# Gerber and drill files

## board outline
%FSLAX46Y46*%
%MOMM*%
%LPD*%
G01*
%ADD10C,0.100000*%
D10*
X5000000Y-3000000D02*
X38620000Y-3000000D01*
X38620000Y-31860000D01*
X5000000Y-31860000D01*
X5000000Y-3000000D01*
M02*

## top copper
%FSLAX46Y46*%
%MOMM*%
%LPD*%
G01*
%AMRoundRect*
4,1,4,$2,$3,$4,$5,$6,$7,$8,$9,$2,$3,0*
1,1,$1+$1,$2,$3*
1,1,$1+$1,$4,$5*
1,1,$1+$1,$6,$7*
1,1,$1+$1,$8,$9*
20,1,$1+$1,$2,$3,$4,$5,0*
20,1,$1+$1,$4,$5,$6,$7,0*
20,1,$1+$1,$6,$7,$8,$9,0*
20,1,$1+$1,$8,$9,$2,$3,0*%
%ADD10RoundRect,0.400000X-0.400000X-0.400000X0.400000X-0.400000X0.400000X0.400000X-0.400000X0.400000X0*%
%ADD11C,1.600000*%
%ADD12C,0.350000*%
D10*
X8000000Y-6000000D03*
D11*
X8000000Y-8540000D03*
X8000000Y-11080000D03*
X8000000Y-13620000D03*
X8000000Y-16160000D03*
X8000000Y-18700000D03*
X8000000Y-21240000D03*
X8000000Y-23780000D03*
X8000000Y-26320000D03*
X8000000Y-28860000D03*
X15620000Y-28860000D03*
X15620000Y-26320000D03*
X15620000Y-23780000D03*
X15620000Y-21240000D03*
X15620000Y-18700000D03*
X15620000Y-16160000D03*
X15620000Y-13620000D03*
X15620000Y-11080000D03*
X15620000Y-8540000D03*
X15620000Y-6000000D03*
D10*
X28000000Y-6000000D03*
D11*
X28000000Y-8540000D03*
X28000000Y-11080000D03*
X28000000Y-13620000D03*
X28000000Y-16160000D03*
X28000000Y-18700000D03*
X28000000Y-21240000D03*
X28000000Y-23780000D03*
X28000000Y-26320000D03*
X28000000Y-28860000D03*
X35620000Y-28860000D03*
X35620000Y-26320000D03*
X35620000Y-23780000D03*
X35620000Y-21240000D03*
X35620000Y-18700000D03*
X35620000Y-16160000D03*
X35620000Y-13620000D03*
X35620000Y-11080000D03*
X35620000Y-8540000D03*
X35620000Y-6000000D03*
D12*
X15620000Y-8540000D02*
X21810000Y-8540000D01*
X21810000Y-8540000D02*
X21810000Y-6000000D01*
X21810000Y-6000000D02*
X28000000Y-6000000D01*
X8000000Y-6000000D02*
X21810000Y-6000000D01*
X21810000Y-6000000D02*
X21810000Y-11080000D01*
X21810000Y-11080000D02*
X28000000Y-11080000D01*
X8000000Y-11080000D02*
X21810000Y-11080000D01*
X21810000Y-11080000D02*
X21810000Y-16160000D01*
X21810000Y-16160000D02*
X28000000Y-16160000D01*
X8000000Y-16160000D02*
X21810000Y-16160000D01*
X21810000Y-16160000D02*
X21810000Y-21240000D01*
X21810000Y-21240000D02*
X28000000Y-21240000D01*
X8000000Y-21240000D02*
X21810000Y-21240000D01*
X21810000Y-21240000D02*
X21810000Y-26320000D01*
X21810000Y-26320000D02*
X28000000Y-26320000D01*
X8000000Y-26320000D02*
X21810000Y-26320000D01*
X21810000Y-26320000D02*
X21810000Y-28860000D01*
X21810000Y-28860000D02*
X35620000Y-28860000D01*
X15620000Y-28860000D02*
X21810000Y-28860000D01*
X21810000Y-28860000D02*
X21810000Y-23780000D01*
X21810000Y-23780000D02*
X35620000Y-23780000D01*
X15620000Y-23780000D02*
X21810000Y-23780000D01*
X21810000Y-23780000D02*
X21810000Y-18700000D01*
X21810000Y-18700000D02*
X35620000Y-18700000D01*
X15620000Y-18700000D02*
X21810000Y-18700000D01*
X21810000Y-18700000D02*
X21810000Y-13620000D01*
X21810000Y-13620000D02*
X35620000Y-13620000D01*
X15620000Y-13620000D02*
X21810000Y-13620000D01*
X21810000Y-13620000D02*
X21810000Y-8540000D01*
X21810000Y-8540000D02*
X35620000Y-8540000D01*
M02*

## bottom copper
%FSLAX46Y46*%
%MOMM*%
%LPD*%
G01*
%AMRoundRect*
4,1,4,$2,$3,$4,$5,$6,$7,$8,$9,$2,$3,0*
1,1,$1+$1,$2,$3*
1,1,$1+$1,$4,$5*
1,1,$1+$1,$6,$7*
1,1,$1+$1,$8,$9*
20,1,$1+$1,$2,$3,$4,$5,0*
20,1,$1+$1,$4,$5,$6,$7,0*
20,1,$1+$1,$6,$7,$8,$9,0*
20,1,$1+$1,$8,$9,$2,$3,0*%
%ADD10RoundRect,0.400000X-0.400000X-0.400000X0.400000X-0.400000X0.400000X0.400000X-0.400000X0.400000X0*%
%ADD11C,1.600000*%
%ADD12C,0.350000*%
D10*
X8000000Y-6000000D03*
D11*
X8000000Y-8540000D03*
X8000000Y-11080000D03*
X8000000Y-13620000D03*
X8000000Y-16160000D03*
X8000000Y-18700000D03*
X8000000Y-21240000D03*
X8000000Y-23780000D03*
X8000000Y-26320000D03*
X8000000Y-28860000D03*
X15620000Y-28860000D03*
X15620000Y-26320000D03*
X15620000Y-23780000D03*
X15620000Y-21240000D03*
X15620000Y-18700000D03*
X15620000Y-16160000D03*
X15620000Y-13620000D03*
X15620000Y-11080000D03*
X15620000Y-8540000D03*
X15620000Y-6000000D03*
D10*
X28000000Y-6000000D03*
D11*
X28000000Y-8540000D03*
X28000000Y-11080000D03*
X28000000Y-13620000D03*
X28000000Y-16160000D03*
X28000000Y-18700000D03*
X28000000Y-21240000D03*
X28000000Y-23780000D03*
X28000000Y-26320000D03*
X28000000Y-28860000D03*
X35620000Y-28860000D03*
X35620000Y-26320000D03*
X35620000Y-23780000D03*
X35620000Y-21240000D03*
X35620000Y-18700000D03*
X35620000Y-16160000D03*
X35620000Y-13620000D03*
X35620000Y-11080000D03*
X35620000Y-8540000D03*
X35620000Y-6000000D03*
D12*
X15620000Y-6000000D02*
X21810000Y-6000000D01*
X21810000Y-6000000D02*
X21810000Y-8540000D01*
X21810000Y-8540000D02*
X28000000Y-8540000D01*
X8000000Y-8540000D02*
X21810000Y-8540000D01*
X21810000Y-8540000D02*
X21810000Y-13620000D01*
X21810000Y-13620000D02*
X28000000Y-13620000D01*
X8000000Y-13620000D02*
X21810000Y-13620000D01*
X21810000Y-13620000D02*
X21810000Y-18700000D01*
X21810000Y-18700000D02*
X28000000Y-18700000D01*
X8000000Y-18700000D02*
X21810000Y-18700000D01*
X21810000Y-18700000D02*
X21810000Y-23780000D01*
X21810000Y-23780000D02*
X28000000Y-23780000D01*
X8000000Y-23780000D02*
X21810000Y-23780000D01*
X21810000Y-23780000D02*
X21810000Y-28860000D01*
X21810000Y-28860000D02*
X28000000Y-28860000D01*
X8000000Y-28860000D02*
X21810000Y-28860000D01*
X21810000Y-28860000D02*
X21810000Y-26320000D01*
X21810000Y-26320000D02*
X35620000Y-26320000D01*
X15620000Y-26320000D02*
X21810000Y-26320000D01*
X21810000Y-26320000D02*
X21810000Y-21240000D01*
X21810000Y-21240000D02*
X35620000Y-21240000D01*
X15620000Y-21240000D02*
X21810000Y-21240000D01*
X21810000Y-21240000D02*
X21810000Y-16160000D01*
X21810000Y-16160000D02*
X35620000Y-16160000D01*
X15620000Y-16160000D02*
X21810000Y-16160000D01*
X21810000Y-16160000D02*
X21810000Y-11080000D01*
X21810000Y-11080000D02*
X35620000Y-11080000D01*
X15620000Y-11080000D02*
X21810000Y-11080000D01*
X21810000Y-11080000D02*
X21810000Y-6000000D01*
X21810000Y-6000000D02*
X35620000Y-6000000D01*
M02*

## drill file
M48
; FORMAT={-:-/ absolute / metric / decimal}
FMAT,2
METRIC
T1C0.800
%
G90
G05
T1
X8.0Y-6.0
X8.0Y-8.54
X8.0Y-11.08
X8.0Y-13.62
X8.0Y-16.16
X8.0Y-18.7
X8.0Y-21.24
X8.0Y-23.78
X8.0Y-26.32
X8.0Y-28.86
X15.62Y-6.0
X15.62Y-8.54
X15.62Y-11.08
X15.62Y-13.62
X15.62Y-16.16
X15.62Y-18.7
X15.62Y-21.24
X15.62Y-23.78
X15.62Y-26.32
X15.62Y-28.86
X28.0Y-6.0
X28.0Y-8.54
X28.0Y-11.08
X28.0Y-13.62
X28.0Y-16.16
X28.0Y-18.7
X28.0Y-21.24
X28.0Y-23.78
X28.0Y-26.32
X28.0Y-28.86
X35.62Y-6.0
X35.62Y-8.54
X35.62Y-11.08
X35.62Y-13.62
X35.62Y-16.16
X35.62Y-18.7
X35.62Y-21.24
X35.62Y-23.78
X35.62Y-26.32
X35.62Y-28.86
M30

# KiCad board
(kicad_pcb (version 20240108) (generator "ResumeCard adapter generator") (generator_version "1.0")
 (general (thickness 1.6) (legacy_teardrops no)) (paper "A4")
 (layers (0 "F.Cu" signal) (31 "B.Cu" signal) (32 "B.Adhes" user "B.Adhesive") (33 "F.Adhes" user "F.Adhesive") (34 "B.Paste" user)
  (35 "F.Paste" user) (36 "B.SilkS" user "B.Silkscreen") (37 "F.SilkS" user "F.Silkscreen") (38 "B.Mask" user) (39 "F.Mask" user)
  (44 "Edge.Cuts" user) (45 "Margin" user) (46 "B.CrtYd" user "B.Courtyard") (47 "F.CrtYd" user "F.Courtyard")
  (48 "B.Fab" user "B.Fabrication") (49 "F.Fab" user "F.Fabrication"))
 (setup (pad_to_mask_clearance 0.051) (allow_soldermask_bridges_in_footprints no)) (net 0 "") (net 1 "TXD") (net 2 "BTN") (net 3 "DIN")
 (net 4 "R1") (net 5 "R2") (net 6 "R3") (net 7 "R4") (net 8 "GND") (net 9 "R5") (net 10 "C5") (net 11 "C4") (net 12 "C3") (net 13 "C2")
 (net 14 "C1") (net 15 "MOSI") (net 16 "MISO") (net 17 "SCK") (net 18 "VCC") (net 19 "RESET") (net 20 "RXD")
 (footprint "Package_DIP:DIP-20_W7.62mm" (layer "F.Cu") (at 8.0 6.0)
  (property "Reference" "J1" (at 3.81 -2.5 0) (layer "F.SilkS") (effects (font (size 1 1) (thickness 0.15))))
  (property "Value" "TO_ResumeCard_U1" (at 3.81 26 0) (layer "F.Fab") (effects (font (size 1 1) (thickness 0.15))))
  (pad "1" thru_hole roundrect (at 0.0 0.0) (size 1.6 1.6) (drill 0.8) (layers "*.Cu" "*.Mask") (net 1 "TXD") (roundrect_rratio 0.25))
  (pad "2" thru_hole circle (at 0.0 2.54) (size 1.6 1.6) (drill 0.8) (layers "*.Cu" "*.Mask") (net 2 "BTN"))
  (pad "3" thru_hole circle (at 0.0 5.08) (size 1.6 1.6) (drill 0.8) (layers "*.Cu" "*.Mask") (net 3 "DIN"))
  (pad "4" thru_hole circle (at 0.0 7.62) (size 1.6 1.6) (drill 0.8) (layers "*.Cu" "*.Mask") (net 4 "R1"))
  (pad "5" thru_hole circle (at 0.0 10.16) (size 1.6 1.6) (drill 0.8) (layers "*.Cu" "*.Mask") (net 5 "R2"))
  (pad "6" thru_hole circle (at 0.0 12.7) (size 1.6 1.6) (drill 0.8) (layers "*.Cu" "*.Mask") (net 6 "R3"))
  (pad "7" thru_hole circle (at 0.0 15.24) (size 1.6 1.6) (drill 0.8) (layers "*.Cu" "*.Mask") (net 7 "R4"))
  (pad "8" thru_hole circle (at 0.0 17.78) (size 1.6 1.6) (drill 0.8) (layers "*.Cu" "*.Mask") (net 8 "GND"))
  (pad "9" thru_hole circle (at 0.0 20.32) (size 1.6 1.6) (drill 0.8) (layers "*.Cu" "*.Mask") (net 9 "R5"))
  (pad "10" thru_hole circle (at 0.0 22.86) (size 1.6 1.6) (drill 0.8) (layers "*.Cu" "*.Mask") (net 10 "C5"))
  (pad "11" thru_hole circle (at 7.62 22.86) (size 1.6 1.6) (drill 0.8) (layers "*.Cu" "*.Mask") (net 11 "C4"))
  (pad "12" thru_hole circle (at 7.62 20.32) (size 1.6 1.6) (drill 0.8) (layers "*.Cu" "*.Mask") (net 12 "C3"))
  (pad "13" thru_hole circle (at 7.62 17.78) (size 1.6 1.6) (drill 0.8) (layers "*.Cu" "*.Mask") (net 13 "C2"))
  (pad "14" thru_hole circle (at 7.62 15.24) (size 1.6 1.6) (drill 0.8) (layers "*.Cu" "*.Mask") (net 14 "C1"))
  (pad "15" thru_hole circle (at 7.62 12.7) (size 1.6 1.6) (drill 0.8) (layers "*.Cu" "*.Mask") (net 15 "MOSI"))
  (pad "16" thru_hole circle (at 7.62 10.16) (size 1.6 1.6) (drill 0.8) (layers "*.Cu" "*.Mask") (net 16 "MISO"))
  (pad "17" thru_hole circle (at 7.62 7.62) (size 1.6 1.6) (drill 0.8) (layers "*.Cu" "*.Mask") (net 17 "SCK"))
  (pad "18" thru_hole circle (at 7.62 5.08) (size 1.6 1.6) (drill 0.8) (layers "*.Cu" "*.Mask") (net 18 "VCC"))
  (pad "19" thru_hole circle (at 7.62 2.54) (size 1.6 1.6) (drill 0.8) (layers "*.Cu" "*.Mask") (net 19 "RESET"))
  (pad "20" thru_hole circle (at 7.62 0.0) (size 1.6 1.6) (drill 0.8) (layers "*.Cu" "*.Mask") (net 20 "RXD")))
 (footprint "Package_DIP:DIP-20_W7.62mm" (layer "F.Cu") (at 28.0 6.0)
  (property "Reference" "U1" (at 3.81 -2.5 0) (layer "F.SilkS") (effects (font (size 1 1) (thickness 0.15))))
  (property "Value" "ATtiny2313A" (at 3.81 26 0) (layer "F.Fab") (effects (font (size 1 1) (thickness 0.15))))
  (pad "1" thru_hole roundrect (at 0.0 0.0) (size 1.6 1.6) (drill 0.8) (layers "*.Cu" "*.Mask") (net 19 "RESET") (roundrect_rratio 0.25))
  (pad "2" thru_hole circle (at 0.0 2.54) (size 1.6 1.6) (drill 0.8) (layers "*.Cu" "*.Mask") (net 20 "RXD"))
  (pad "3" thru_hole circle (at 0.0 5.08) (size 1.6 1.6) (drill 0.8) (layers "*.Cu" "*.Mask") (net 1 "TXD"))
  (pad "4" thru_hole circle (at 0.0 7.62) (size 1.6 1.6) (drill 0.8) (layers "*.Cu" "*.Mask") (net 2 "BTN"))
  (pad "5" thru_hole circle (at 0.0 10.16) (size 1.6 1.6) (drill 0.8) (layers "*.Cu" "*.Mask") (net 3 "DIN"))
  (pad "6" thru_hole circle (at 0.0 12.7) (size 1.6 1.6) (drill 0.8) (layers "*.Cu" "*.Mask") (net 4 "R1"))
  (pad "7" thru_hole circle (at 0.0 15.24) (size 1.6 1.6) (drill 0.8) (layers "*.Cu" "*.Mask") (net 5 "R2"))
  (pad "8" thru_hole circle (at 0.0 17.78) (size 1.6 1.6) (drill 0.8) (layers "*.Cu" "*.Mask") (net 6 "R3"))
  (pad "9" thru_hole circle (at 0.0 20.32) (size 1.6 1.6) (drill 0.8) (layers "*.Cu" "*.Mask") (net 7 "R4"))
  (pad "10" thru_hole circle (at 0.0 22.86) (size 1.6 1.6) (drill 0.8) (layers "*.Cu" "*.Mask") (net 8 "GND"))
  (pad "11" thru_hole circle (at 7.62 22.86) (size 1.6 1.6) (drill 0.8) (layers "*.Cu" "*.Mask") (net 9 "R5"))
  (pad "12" thru_hole circle (at 7.62 20.32) (size 1.6 1.6) (drill 0.8) (layers "*.Cu" "*.Mask") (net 10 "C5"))
  (pad "13" thru_hole circle (at 7.62 17.78) (size 1.6 1.6) (drill 0.8) (layers "*.Cu" "*.Mask") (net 11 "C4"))
  (pad "14" thru_hole circle (at 7.62 15.24) (size 1.6 1.6) (drill 0.8) (layers "*.Cu" "*.Mask") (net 12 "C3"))
  (pad "15" thru_hole circle (at 7.62 12.7) (size 1.6 1.6) (drill 0.8) (layers "*.Cu" "*.Mask") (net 13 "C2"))
  (pad "16" thru_hole circle (at 7.62 10.16) (size 1.6 1.6) (drill 0.8) (layers "*.Cu" "*.Mask") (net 14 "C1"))
  (pad "17" thru_hole circle (at 7.62 7.62) (size 1.6 1.6) (drill 0.8) (layers "*.Cu" "*.Mask") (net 15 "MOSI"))
  (pad "18" thru_hole circle (at 7.62 5.08) (size 1.6 1.6) (drill 0.8) (layers "*.Cu" "*.Mask") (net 16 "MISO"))
  (pad "19" thru_hole circle (at 7.62 2.54) (size 1.6 1.6) (drill 0.8) (layers "*.Cu" "*.Mask") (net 17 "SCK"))
  (pad "20" thru_hole circle (at 7.62 0.0) (size 1.6 1.6) (drill 0.8) (layers "*.Cu" "*.Mask") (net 18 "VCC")))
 (segment (start 15.620 8.540) (end 21.810 8.540) (width 0.35) (layer "F.Cu") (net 19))
 (segment (start 21.810 8.540) (end 21.810 6.000) (width 0.35) (layer "F.Cu") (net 19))
 (segment (start 21.810 6.000) (end 28.000 6.000) (width 0.35) (layer "F.Cu") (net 19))
 (segment (start 15.620 6.000) (end 21.810 6.000) (width 0.35) (layer "B.Cu") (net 20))
 (segment (start 21.810 6.000) (end 21.810 8.540) (width 0.35) (layer "B.Cu") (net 20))
 (segment (start 21.810 8.540) (end 28.000 8.540) (width 0.35) (layer "B.Cu") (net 20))
 (segment (start 8.000 6.000) (end 21.810 6.000) (width 0.35) (layer "F.Cu") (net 1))
 (segment (start 21.810 6.000) (end 21.810 11.080) (width 0.35) (layer "F.Cu") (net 1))
 (segment (start 21.810 11.080) (end 28.000 11.080) (width 0.35) (layer "F.Cu") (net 1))
 (segment (start 8.000 8.540) (end 21.810 8.540) (width 0.35) (layer "B.Cu") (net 2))
 (segment (start 21.810 8.540) (end 21.810 13.620) (width 0.35) (layer "B.Cu") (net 2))
 (segment (start 21.810 13.620) (end 28.000 13.620) (width 0.35) (layer "B.Cu") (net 2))
 (segment (start 8.000 11.080) (end 21.810 11.080) (width 0.35) (layer "F.Cu") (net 3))
 (segment (start 21.810 11.080) (end 21.810 16.160) (width 0.35) (layer "F.Cu") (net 3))
 (segment (start 21.810 16.160) (end 28.000 16.160) (width 0.35) (layer "F.Cu") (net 3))
 (segment (start 8.000 13.620) (end 21.810 13.620) (width 0.35) (layer "B.Cu") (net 4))
 (segment (start 21.810 13.620) (end 21.810 18.700) (width 0.35) (layer "B.Cu") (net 4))
 (segment (start 21.810 18.700) (end 28.000 18.700) (width 0.35) (layer "B.Cu") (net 4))
 (segment (start 8.000 16.160) (end 21.810 16.160) (width 0.35) (layer "F.Cu") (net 5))
 (segment (start 21.810 16.160) (end 21.810 21.240) (width 0.35) (layer "F.Cu") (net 5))
 (segment (start 21.810 21.240) (end 28.000 21.240) (width 0.35) (layer "F.Cu") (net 5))
 (segment (start 8.000 18.700) (end 21.810 18.700) (width 0.35) (layer "B.Cu") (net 6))
 (segment (start 21.810 18.700) (end 21.810 23.780) (width 0.35) (layer "B.Cu") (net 6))
 (segment (start 21.810 23.780) (end 28.000 23.780) (width 0.35) (layer "B.Cu") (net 6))
 (segment (start 8.000 21.240) (end 21.810 21.240) (width 0.35) (layer "F.Cu") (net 7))
 (segment (start 21.810 21.240) (end 21.810 26.320) (width 0.35) (layer "F.Cu") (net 7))
 (segment (start 21.810 26.320) (end 28.000 26.320) (width 0.35) (layer "F.Cu") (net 7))
 (segment (start 8.000 23.780) (end 21.810 23.780) (width 0.35) (layer "B.Cu") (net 8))
 (segment (start 21.810 23.780) (end 21.810 28.860) (width 0.35) (layer "B.Cu") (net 8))
 (segment (start 21.810 28.860) (end 28.000 28.860) (width 0.35) (layer "B.Cu") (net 8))
 (segment (start 8.000 26.320) (end 21.810 26.320) (width 0.35) (layer "F.Cu") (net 9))
 (segment (start 21.810 26.320) (end 21.810 28.860) (width 0.35) (layer "F.Cu") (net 9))
 (segment (start 21.810 28.860) (end 35.620 28.860) (width 0.35) (layer "F.Cu") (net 9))
 (segment (start 8.000 28.860) (end 21.810 28.860) (width 0.35) (layer "B.Cu") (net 10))
 (segment (start 21.810 28.860) (end 21.810 26.320) (width 0.35) (layer "B.Cu") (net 10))
 (segment (start 21.810 26.320) (end 35.620 26.320) (width 0.35) (layer "B.Cu") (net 10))
 (segment (start 15.620 28.860) (end 21.810 28.860) (width 0.35) (layer "F.Cu") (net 11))
 (segment (start 21.810 28.860) (end 21.810 23.780) (width 0.35) (layer "F.Cu") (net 11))
 (segment (start 21.810 23.780) (end 35.620 23.780) (width 0.35) (layer "F.Cu") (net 11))
 (segment (start 15.620 26.320) (end 21.810 26.320) (width 0.35) (layer "B.Cu") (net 12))
 (segment (start 21.810 26.320) (end 21.810 21.240) (width 0.35) (layer "B.Cu") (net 12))
 (segment (start 21.810 21.240) (end 35.620 21.240) (width 0.35) (layer "B.Cu") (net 12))
 (segment (start 15.620 23.780) (end 21.810 23.780) (width 0.35) (layer "F.Cu") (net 13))
 (segment (start 21.810 23.780) (end 21.810 18.700) (width 0.35) (layer "F.Cu") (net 13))
 (segment (start 21.810 18.700) (end 35.620 18.700) (width 0.35) (layer "F.Cu") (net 13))
 (segment (start 15.620 21.240) (end 21.810 21.240) (width 0.35) (layer "B.Cu") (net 14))
 (segment (start 21.810 21.240) (end 21.810 16.160) (width 0.35) (layer "B.Cu") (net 14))
 (segment (start 21.810 16.160) (end 35.620 16.160) (width 0.35) (layer "B.Cu") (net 14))
 (segment (start 15.620 18.700) (end 21.810 18.700) (width 0.35) (layer "F.Cu") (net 15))
 (segment (start 21.810 18.700) (end 21.810 13.620) (width 0.35) (layer "F.Cu") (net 15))
 (segment (start 21.810 13.620) (end 35.620 13.620) (width 0.35) (layer "F.Cu") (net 15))
 (segment (start 15.620 16.160) (end 21.810 16.160) (width 0.35) (layer "B.Cu") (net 16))
 (segment (start 21.810 16.160) (end 21.810 11.080) (width 0.35) (layer "B.Cu") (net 16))
 (segment (start 21.810 11.080) (end 35.620 11.080) (width 0.35) (layer "B.Cu") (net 16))
 (segment (start 15.620 13.620) (end 21.810 13.620) (width 0.35) (layer "F.Cu") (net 17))
 (segment (start 21.810 13.620) (end 21.810 8.540) (width 0.35) (layer "F.Cu") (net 17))
 (segment (start 21.810 8.540) (end 35.620 8.540) (width 0.35) (layer "F.Cu") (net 17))
 (segment (start 15.620 11.080) (end 21.810 11.080) (width 0.35) (layer "B.Cu") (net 18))
 (segment (start 21.810 11.080) (end 21.810 6.000) (width 0.35) (layer "B.Cu") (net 18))
 (segment (start 21.810 6.000) (end 35.620 6.000) (width 0.35) (layer "B.Cu") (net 18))
 (gr_rect (start 5.000 3.000) (end 38.620 31.860) (stroke (width 0.1) (type solid)) (fill none) (layer "Edge.Cuts")))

